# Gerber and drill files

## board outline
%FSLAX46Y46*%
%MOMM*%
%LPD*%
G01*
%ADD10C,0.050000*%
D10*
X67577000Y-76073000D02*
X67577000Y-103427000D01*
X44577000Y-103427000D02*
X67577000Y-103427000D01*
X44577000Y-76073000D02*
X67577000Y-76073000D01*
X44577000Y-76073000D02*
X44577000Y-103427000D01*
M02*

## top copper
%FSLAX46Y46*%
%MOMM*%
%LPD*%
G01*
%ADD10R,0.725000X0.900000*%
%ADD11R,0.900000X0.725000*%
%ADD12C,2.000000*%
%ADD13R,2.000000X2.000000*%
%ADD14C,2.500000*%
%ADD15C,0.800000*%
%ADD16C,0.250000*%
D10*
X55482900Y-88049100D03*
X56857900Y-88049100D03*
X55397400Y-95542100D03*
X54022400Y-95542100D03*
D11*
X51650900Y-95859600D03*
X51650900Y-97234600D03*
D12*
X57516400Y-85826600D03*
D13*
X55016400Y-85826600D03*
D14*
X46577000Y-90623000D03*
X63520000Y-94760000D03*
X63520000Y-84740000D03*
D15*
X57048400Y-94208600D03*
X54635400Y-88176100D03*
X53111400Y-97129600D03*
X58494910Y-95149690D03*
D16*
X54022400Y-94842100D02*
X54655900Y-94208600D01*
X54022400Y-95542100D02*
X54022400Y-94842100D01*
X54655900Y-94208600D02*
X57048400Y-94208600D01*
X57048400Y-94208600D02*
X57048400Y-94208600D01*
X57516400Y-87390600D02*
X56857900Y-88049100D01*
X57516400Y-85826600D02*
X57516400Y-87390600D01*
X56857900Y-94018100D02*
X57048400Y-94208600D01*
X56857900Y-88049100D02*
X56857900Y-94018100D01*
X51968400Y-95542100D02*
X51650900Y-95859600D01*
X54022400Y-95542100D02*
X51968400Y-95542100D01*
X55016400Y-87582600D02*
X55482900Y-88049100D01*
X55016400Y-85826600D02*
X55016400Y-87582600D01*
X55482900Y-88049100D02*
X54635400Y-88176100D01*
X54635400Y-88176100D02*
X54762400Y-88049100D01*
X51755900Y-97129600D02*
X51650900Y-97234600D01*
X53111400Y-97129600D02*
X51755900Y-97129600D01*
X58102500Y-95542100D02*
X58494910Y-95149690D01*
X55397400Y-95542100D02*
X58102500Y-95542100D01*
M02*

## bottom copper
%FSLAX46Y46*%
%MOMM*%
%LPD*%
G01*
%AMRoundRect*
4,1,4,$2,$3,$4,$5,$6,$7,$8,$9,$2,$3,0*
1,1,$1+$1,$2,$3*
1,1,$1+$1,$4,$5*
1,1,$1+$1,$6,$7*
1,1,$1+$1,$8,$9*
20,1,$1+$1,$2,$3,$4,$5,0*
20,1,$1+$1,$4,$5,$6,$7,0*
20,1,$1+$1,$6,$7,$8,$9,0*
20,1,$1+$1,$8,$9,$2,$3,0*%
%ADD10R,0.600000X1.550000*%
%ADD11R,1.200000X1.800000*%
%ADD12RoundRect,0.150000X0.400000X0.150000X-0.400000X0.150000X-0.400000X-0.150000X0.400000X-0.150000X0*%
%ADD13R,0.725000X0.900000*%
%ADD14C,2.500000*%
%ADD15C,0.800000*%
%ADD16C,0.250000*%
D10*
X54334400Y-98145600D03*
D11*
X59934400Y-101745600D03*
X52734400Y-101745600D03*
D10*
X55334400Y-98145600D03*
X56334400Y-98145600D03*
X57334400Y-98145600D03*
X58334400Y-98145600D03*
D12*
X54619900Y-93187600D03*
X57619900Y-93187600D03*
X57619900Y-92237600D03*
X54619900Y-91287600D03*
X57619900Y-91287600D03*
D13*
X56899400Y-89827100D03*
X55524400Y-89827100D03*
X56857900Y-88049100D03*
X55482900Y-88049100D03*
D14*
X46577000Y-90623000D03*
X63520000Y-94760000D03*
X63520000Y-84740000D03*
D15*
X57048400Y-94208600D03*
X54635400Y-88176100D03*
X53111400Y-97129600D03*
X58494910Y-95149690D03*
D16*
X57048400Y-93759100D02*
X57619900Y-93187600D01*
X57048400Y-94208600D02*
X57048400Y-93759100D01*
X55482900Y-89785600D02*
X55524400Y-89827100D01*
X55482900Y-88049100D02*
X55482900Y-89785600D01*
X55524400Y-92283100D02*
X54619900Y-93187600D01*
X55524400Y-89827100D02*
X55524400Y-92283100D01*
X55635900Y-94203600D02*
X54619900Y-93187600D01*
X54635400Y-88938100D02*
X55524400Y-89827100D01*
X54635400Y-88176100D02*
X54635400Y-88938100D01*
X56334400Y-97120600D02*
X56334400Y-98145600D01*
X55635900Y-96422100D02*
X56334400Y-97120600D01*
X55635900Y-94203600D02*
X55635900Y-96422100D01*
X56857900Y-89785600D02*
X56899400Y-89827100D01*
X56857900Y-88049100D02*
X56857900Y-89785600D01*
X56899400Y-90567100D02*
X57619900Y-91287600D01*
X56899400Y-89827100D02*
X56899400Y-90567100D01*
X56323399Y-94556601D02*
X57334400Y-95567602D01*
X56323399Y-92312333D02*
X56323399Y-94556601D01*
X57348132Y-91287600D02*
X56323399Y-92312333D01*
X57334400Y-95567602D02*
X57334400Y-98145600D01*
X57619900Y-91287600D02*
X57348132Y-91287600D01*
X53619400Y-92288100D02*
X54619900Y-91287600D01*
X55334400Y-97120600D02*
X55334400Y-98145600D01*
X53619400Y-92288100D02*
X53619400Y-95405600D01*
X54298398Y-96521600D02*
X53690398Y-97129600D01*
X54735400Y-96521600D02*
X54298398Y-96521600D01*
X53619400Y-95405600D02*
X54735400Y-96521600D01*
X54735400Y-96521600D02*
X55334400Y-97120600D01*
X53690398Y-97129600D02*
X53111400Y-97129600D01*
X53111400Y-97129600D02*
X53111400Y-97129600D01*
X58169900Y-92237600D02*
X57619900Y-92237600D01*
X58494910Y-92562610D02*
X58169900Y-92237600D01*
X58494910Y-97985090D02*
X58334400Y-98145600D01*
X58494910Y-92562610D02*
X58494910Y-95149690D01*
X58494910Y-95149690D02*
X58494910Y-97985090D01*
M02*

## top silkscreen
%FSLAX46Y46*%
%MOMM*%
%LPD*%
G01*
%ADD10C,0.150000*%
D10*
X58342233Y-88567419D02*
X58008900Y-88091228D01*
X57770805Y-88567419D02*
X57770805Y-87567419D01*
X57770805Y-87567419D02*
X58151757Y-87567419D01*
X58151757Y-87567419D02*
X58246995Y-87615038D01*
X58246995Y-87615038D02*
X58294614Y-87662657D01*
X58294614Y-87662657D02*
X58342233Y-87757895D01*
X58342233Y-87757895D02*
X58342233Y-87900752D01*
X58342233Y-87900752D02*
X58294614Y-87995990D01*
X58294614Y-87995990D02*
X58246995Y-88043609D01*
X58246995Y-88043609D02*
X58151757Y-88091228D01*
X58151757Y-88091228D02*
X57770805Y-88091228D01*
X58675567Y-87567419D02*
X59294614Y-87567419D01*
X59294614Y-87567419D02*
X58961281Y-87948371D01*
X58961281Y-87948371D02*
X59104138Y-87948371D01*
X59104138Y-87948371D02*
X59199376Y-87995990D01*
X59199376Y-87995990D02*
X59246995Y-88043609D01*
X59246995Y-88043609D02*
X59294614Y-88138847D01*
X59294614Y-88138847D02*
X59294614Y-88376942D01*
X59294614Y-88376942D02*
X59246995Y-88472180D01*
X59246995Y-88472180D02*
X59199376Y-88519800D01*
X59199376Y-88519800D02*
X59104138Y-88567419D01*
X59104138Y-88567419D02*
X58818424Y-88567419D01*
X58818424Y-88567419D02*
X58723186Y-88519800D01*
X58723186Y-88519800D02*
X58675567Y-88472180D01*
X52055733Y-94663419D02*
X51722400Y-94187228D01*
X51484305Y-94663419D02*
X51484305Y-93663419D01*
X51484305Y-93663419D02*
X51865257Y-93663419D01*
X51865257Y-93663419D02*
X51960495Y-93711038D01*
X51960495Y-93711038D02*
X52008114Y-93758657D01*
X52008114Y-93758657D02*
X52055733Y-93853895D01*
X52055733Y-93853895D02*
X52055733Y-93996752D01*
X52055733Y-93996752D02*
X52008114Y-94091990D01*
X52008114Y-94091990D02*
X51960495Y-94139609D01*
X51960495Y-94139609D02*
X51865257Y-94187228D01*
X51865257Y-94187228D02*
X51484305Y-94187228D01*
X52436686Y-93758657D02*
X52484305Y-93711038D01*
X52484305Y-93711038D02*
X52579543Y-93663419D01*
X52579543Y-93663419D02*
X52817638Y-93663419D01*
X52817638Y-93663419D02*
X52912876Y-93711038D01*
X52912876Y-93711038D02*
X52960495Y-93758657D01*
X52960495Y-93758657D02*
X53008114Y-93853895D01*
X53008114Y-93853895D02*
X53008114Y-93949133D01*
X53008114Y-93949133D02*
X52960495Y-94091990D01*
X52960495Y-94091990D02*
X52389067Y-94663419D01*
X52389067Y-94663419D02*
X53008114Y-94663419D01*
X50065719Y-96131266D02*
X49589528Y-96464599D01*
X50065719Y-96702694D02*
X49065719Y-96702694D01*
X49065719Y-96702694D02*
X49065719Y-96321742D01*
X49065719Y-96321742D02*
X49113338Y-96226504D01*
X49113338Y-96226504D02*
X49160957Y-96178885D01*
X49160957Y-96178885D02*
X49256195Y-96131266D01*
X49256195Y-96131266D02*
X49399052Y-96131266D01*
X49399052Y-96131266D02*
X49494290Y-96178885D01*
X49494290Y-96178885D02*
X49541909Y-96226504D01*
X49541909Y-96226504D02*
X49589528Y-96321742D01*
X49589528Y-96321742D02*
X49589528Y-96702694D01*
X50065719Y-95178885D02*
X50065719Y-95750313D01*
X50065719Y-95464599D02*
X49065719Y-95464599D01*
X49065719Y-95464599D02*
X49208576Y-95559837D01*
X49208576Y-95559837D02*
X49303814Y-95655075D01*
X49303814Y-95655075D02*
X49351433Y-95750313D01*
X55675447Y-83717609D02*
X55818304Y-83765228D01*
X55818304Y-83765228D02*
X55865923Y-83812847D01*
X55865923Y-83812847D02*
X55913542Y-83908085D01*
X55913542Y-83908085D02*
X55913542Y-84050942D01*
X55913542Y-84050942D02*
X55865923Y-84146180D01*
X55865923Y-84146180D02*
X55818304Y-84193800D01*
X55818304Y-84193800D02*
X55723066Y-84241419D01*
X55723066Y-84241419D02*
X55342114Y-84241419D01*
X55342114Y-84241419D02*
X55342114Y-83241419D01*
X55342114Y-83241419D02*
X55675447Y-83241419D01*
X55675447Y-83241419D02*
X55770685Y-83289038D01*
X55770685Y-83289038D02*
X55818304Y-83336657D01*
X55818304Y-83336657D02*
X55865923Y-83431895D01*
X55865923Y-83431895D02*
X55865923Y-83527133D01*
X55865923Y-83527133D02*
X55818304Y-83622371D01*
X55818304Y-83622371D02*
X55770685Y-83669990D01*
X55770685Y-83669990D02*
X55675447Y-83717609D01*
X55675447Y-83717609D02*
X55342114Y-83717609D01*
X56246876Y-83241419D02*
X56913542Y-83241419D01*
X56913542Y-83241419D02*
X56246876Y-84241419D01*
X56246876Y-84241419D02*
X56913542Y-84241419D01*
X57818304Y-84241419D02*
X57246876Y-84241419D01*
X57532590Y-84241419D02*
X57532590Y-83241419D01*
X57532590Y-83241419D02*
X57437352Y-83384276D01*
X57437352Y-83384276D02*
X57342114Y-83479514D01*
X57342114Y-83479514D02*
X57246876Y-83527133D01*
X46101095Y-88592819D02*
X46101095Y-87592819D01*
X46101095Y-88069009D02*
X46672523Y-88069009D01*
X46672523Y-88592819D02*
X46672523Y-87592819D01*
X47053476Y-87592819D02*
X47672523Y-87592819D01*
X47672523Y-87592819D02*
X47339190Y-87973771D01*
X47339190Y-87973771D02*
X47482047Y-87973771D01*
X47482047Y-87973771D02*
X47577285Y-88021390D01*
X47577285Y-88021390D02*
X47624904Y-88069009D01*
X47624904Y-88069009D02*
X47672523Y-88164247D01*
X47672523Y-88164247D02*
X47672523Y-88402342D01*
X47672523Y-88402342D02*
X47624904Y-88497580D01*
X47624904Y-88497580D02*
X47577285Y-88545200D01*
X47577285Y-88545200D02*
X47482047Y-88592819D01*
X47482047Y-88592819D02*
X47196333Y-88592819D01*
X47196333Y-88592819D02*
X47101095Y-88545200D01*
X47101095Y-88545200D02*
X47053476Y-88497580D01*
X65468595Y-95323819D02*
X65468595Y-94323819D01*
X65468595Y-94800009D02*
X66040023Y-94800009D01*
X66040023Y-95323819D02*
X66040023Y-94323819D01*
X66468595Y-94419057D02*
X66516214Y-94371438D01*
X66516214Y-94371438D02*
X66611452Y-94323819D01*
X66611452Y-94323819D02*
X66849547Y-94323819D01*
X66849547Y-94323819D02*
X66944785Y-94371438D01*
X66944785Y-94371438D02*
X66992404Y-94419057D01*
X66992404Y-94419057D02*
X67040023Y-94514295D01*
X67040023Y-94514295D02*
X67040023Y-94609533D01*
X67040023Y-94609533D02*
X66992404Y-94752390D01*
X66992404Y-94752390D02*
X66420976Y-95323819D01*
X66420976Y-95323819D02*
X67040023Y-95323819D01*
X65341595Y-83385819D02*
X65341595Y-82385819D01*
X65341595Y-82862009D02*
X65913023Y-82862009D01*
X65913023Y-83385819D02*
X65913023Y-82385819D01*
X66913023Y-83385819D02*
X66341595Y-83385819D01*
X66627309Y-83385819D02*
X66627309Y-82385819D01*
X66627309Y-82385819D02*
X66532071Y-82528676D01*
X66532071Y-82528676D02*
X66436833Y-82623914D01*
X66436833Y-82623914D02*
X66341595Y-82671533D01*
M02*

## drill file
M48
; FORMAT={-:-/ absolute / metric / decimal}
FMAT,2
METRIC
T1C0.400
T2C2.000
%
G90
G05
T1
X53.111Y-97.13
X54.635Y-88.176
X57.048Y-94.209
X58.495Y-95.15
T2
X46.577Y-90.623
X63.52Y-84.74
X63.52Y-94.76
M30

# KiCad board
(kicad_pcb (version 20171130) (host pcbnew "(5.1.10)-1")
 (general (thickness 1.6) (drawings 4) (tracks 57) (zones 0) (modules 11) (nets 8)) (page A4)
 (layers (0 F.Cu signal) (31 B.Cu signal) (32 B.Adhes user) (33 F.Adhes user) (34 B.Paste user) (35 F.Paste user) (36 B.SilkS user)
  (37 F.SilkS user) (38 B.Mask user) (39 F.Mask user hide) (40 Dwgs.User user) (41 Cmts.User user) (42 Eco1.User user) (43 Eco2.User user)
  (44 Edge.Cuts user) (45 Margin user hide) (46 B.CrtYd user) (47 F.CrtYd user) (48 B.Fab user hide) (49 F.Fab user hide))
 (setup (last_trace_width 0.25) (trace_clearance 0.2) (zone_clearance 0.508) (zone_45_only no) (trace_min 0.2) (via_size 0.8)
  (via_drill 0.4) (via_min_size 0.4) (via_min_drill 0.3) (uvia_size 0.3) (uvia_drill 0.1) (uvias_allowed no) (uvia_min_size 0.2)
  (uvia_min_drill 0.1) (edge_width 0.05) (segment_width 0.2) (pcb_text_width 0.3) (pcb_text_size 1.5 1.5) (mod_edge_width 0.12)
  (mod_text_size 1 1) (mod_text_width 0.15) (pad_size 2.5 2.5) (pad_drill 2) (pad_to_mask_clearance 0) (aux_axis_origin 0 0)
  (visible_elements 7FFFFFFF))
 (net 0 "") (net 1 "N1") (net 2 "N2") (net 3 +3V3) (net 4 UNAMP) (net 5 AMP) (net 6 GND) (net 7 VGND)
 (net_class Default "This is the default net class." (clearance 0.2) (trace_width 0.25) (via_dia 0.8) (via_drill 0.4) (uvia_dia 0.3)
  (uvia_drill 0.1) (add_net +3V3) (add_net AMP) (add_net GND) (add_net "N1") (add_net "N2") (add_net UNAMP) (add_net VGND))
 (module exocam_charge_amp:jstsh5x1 (layer B.Cu) (at 55.5244 95.6056 180)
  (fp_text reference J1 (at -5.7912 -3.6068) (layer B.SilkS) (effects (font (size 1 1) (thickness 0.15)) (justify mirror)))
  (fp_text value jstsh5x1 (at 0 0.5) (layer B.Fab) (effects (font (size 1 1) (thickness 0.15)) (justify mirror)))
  (pad 5 smd rect (at 1.19 -2.54 180) (size 0.6 1.55) (layers B.Cu B.Paste B.Mask) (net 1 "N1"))
  (pad 6 smd rect (at -4.41 -6.14 180) (size 1.2 1.8) (layers B.Cu B.Paste B.Mask) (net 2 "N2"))
  (pad 6 smd rect (at 2.79 -6.14 180) (size 1.2 1.8) (layers B.Cu B.Paste B.Mask) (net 2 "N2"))
  (pad 4 smd rect (at 0.19 -2.54 180) (size 0.6 1.55) (layers B.Cu B.Paste B.Mask) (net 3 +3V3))
  (pad 3 smd rect (at -0.81 -2.54 180) (size 0.6 1.55) (layers B.Cu B.Paste B.Mask) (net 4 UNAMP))
  (pad 2 smd rect (at -1.81 -2.54 180) (size 0.6 1.55) (layers B.Cu B.Paste B.Mask) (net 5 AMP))
  (pad 1 smd rect (at -2.81 -2.54 180) (size 0.6 1.55) (layers B.Cu B.Paste B.Mask) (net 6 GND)))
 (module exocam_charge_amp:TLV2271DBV (layer B.Cu) (at 56.3499 88.7476 180)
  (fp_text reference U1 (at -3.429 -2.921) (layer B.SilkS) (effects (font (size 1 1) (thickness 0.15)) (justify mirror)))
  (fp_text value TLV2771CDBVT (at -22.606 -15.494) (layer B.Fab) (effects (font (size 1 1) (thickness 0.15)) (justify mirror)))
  (pad 4 smd roundrect (at 1.73 -4.44 180) (size 1.1 0.6) (layers B.Cu B.Paste B.Mask) (roundrect_rratio 0.25) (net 4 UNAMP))
  (pad 3 smd roundrect (at -1.27 -4.44 180) (size 1.1 0.6) (layers B.Cu B.Paste B.Mask) (roundrect_rratio 0.25) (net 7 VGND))
  (pad 2 smd roundrect (at -1.27 -3.49 180) (size 1.1 0.6) (layers B.Cu B.Paste B.Mask) (roundrect_rratio 0.25) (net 6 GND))
  (pad 5 smd roundrect (at 1.73 -2.54 180) (size 1.1 0.6) (layers B.Cu B.Paste B.Mask) (roundrect_rratio 0.25) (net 3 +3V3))
  (pad 1 smd roundrect (at -1.27 -2.54 180) (size 1.1 0.6) (layers B.Cu B.Paste B.Mask) (roundrect_rratio 0.25) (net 5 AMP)))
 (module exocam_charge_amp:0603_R (layer B.Cu) (at 56.7944 92.3671)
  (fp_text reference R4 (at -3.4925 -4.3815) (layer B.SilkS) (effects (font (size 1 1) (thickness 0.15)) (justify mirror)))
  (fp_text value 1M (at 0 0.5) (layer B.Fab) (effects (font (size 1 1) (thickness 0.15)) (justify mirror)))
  (pad 2 smd rect (at 0.105 -2.54) (size 0.725 0.9) (layers B.Cu B.Paste B.Mask) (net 5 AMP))
  (pad 1 smd rect (at -1.27 -2.54) (size 0.725 0.9) (layers B.Cu B.Paste B.Mask) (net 4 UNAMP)))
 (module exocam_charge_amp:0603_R (layer F.Cu) (at 55.5879 90.5891 180)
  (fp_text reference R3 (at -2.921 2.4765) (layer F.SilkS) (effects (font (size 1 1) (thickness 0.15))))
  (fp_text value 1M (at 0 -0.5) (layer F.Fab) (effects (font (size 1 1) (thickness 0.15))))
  (pad 2 smd rect (at 0.105 2.54 180) (size 0.725 0.9) (layers F.Cu F.Paste F.Mask) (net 4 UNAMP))
  (pad 1 smd rect (at -1.27 2.54 180) (size 0.725 0.9) (layers F.Cu F.Paste F.Mask) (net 7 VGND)))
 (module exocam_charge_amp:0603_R (layer F.Cu) (at 55.2924 93.0021)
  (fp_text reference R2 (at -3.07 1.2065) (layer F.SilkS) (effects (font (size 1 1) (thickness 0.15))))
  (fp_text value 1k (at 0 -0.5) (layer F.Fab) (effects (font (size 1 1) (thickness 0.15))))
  (pad 2 smd rect (at 0.105 2.54) (size 0.725 0.9) (layers F.Cu F.Paste F.Mask) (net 6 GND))
  (pad 1 smd rect (at -1.27 2.54) (size 0.725 0.9) (layers F.Cu F.Paste F.Mask) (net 7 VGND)))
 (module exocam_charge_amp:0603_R (layer F.Cu) (at 49.1109 95.9646 90)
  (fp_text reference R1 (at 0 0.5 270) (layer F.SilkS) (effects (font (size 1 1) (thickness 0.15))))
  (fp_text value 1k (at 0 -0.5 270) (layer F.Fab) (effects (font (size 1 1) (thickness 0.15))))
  (pad 2 smd rect (at 0.105 2.54 90) (size 0.725 0.9) (layers F.Cu F.Paste F.Mask) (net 7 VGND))
  (pad 1 smd rect (at -1.27 2.54 90) (size 0.725 0.9) (layers F.Cu F.Paste F.Mask) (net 3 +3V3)))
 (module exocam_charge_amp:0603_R (layer B.Cu) (at 56.7529 90.5891)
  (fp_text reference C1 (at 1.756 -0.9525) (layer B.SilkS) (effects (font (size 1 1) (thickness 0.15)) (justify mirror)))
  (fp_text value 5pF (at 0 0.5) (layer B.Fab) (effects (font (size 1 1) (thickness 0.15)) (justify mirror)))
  (pad 2 smd rect (at 0.105 -2.54) (size 0.725 0.9) (layers B.Cu B.Paste B.Mask) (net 5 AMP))
  (pad 1 smd rect (at -1.27 -2.54) (size 0.725 0.9) (layers B.Cu B.Paste B.Mask) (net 4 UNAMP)))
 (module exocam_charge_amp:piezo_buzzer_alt (layer F.Cu) (at 56.5564 83.2866)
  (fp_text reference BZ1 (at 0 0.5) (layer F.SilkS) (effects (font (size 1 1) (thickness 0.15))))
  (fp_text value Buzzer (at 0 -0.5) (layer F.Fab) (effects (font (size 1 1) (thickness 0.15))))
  (pad 2 smd circle (at 0.96 2.54) (size 2 2) (layers F.Cu F.Paste F.Mask) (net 7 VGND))
  (pad 1 smd rect (at -1.54 2.54) (size 2 2) (layers F.Cu F.Paste F.Mask) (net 4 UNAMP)))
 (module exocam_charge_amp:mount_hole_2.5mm (layer F.Cu) (at 60.1815 91.44)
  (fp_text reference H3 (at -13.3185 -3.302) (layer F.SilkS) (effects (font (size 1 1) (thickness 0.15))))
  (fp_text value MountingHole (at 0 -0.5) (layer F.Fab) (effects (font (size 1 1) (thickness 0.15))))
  (pad 1 thru_hole circle (at -13.6045 -0.817) (size 2.5 2.5) (drill 2) (layers *.Cu *.Mask)))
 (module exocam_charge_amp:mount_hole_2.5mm (layer F.Cu) (at 48.7045 94.9325)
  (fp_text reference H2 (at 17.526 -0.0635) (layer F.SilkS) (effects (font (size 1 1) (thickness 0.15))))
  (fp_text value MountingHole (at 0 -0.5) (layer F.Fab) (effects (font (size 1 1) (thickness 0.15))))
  (pad 1 thru_hole circle (at 14.8155 -0.1725) (size 2.5 2.5) (drill 2) (layers *.Cu *.Mask)))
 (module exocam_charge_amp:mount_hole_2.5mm (layer F.Cu) (at 48.641 75.565)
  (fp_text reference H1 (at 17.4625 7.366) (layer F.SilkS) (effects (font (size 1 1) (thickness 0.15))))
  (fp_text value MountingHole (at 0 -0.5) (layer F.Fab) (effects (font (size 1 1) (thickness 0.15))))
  (pad 1 thru_hole circle (at 14.879 9.175) (size 2.5 2.5) (drill 2) (layers *.Cu *.Mask)))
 (gr_line (start 67.577 76.073) (end 67.577 103.427) (layer Edge.Cuts) (width 0.05))
 (gr_line (start 44.577 103.427) (end 67.577 103.427) (layer Edge.Cuts) (width 0.05))
 (gr_line (start 44.577 76.073) (end 67.577 76.073) (layer Edge.Cuts) (width 0.05))
 (gr_line (start 44.577 76.073) (end 44.577 103.427) (layer Edge.Cuts) (width 0.05))
 (segment (start 54.0224 94.8421) (end 54.6559 94.2086) (width 0.25) (layer F.Cu) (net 7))
 (segment (start 54.0224 95.5421) (end 54.0224 94.8421) (width 0.25) (layer F.Cu) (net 7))
 (segment (start 54.6559 94.2086) (end 57.0484 94.2086) (width 0.25) (layer F.Cu) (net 7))
 (segment (start 57.0484 94.2086) (end 57.0484 94.2086) (width 0.25) (layer F.Cu) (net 7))
 (via (at 57.0484 94.2086) (size 0.8) (drill 0.4) (layers F.Cu B.Cu) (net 7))
 (segment (start 57.0484 93.7591) (end 57.6199 93.1876) (width 0.25) (layer B.Cu) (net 7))
 (segment (start 57.0484 94.2086) (end 57.0484 93.7591) (width 0.25) (layer B.Cu) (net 7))
 (segment (start 57.5164 87.3906) (end 56.8579 88.0491) (width 0.25) (layer F.Cu) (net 7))
 (segment (start 57.5164 85.8266) (end 57.5164 87.3906) (width 0.25) (layer F.Cu) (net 7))
 (segment (start 56.8579 94.0181) (end 57.0484 94.2086) (width 0.25) (layer F.Cu) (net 7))
 (segment (start 56.8579 88.0491) (end 56.8579 94.0181) (width 0.25) (layer F.Cu) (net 7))
 (segment (start 51.9684 95.5421) (end 51.6509 95.8596) (width 0.25) (layer F.Cu) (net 7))
 (segment (start 54.0224 95.5421) (end 51.9684 95.5421) (width 0.25) (layer F.Cu) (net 7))
 (segment (start 55.4829 89.7856) (end 55.5244 89.8271) (width 0.25) (layer B.Cu) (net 4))
 (segment (start 55.4829 88.0491) (end 55.4829 89.7856) (width 0.25) (layer B.Cu) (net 4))
 (segment (start 55.5244 92.2831) (end 54.6199 93.1876) (width 0.25) (layer B.Cu) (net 4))
 (segment (start 55.5244 89.8271) (end 55.5244 92.2831) (width 0.25) (layer B.Cu) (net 4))
 (segment (start 55.6359 94.2036) (end 54.6199 93.1876) (width 0.25) (layer B.Cu) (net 4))
 (segment (start 55.0164 87.5826) (end 55.4829 88.0491) (width 0.25) (layer F.Cu) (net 4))
 (segment (start 55.0164 85.8266) (end 55.0164 87.5826) (width 0.25) (layer F.Cu) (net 4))
 (segment (start 55.4829 88.0491) (end 54.6354 88.1761) (width 0.25) (layer F.Cu) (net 4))
 (segment (start 54.6354 88.1761) (end 54.7624 88.0491) (width 0.25) (layer F.Cu) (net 4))
 (via (at 54.6354 88.1761) (size 0.8) (drill 0.4) (layers F.Cu B.Cu) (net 4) (status 1000000))
 (segment (start 54.6354 88.9381) (end 55.5244 89.8271) (width 0.25) (layer B.Cu) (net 4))
 (segment (start 54.6354 88.1761) (end 54.6354 88.9381) (width 0.25) (layer B.Cu) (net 4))
 (segment (start 56.3344 97.1206) (end 56.3344 98.1456) (width 0.25) (layer B.Cu) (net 4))
 (segment (start 55.6359 96.4221) (end 56.3344 97.1206) (width 0.25) (layer B.Cu) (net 4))
 (segment (start 55.6359 94.2036) (end 55.6359 96.4221) (width 0.25) (layer B.Cu) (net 4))
 (segment (start 56.8579 89.7856) (end 56.8994 89.8271) (width 0.25) (layer B.Cu) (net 5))
 (segment (start 56.8579 88.0491) (end 56.8579 89.7856) (width 0.25) (layer B.Cu) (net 5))
 (segment (start 56.8994 90.5671) (end 57.6199 91.2876) (width 0.25) (layer B.Cu) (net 5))
 (segment (start 56.8994 89.8271) (end 56.8994 90.5671) (width 0.25) (layer B.Cu) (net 5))
 (segment (start 56.323399 94.556601) (end 57.3344 95.567602) (width 0.25) (layer B.Cu) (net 5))
 (segment (start 56.323399 92.312333) (end 56.323399 94.556601) (width 0.25) (layer B.Cu) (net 5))
 (segment (start 57.348132 91.2876) (end 56.323399 92.312333) (width 0.25) (layer B.Cu) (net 5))
 (segment (start 57.3344 95.567602) (end 57.3344 98.1456) (width 0.25) (layer B.Cu) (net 5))
 (segment (start 57.6199 91.2876) (end 57.348132 91.2876) (width 0.25) (layer B.Cu) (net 5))
 (segment (start 53.6194 92.2881) (end 54.6199 91.2876) (width 0.25) (layer B.Cu) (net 3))
 (segment (start 55.3344 97.1206) (end 55.3344 98.1456) (width 0.25) (layer B.Cu) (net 3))
 (segment (start 53.6194 92.2881) (end 53.6194 95.4056) (width 0.25) (layer B.Cu) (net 3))
 (segment (start 54.298398 96.5216) (end 53.690398 97.1296) (width 0.25) (layer B.Cu) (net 3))
 (segment (start 54.7354 96.5216) (end 54.298398 96.5216) (width 0.25) (layer B.Cu) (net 3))
 (segment (start 53.6194 95.4056) (end 54.7354 96.5216) (width 0.25) (layer B.Cu) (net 3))
 (segment (start 54.7354 96.5216) (end 55.3344 97.1206) (width 0.25) (layer B.Cu) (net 3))
 (segment (start 53.690398 97.1296) (end 53.1114 97.1296) (width 0.25) (layer B.Cu) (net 3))
 (segment (start 53.1114 97.1296) (end 53.1114 97.1296) (width 0.25) (layer B.Cu) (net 3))
 (via (at 53.1114 97.1296) (size 0.8) (drill 0.4) (layers F.Cu B.Cu) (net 3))
 (segment (start 51.7559 97.1296) (end 51.6509 97.2346) (width 0.25) (layer F.Cu) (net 3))
 (segment (start 53.1114 97.1296) (end 51.7559 97.1296) (width 0.25) (layer F.Cu) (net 3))
 (segment (start 58.1699 92.2376) (end 57.6199 92.2376) (width 0.25) (layer B.Cu) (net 6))
 (segment (start 58.49491 92.56261) (end 58.1699 92.2376) (width 0.25) (layer B.Cu) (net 6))
 (segment (start 58.49491 97.98509) (end 58.3344 98.1456) (width 0.25) (layer B.Cu) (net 6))
 (segment (start 58.49491 92.56261) (end 58.49491 95.14969) (width 0.25) (layer B.Cu) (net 6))
 (segment (start 58.49491 95.14969) (end 58.49491 97.98509) (width 0.25) (layer B.Cu) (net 6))
 (via (at 58.49491 95.14969) (size 0.8) (drill 0.4) (layers F.Cu B.Cu) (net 6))
 (segment (start 58.1025 95.5421) (end 58.49491 95.14969) (width 0.25) (layer F.Cu) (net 6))
 (segment (start 55.3974 95.5421) (end 58.1025 95.5421) (width 0.25) (layer F.Cu) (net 6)))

